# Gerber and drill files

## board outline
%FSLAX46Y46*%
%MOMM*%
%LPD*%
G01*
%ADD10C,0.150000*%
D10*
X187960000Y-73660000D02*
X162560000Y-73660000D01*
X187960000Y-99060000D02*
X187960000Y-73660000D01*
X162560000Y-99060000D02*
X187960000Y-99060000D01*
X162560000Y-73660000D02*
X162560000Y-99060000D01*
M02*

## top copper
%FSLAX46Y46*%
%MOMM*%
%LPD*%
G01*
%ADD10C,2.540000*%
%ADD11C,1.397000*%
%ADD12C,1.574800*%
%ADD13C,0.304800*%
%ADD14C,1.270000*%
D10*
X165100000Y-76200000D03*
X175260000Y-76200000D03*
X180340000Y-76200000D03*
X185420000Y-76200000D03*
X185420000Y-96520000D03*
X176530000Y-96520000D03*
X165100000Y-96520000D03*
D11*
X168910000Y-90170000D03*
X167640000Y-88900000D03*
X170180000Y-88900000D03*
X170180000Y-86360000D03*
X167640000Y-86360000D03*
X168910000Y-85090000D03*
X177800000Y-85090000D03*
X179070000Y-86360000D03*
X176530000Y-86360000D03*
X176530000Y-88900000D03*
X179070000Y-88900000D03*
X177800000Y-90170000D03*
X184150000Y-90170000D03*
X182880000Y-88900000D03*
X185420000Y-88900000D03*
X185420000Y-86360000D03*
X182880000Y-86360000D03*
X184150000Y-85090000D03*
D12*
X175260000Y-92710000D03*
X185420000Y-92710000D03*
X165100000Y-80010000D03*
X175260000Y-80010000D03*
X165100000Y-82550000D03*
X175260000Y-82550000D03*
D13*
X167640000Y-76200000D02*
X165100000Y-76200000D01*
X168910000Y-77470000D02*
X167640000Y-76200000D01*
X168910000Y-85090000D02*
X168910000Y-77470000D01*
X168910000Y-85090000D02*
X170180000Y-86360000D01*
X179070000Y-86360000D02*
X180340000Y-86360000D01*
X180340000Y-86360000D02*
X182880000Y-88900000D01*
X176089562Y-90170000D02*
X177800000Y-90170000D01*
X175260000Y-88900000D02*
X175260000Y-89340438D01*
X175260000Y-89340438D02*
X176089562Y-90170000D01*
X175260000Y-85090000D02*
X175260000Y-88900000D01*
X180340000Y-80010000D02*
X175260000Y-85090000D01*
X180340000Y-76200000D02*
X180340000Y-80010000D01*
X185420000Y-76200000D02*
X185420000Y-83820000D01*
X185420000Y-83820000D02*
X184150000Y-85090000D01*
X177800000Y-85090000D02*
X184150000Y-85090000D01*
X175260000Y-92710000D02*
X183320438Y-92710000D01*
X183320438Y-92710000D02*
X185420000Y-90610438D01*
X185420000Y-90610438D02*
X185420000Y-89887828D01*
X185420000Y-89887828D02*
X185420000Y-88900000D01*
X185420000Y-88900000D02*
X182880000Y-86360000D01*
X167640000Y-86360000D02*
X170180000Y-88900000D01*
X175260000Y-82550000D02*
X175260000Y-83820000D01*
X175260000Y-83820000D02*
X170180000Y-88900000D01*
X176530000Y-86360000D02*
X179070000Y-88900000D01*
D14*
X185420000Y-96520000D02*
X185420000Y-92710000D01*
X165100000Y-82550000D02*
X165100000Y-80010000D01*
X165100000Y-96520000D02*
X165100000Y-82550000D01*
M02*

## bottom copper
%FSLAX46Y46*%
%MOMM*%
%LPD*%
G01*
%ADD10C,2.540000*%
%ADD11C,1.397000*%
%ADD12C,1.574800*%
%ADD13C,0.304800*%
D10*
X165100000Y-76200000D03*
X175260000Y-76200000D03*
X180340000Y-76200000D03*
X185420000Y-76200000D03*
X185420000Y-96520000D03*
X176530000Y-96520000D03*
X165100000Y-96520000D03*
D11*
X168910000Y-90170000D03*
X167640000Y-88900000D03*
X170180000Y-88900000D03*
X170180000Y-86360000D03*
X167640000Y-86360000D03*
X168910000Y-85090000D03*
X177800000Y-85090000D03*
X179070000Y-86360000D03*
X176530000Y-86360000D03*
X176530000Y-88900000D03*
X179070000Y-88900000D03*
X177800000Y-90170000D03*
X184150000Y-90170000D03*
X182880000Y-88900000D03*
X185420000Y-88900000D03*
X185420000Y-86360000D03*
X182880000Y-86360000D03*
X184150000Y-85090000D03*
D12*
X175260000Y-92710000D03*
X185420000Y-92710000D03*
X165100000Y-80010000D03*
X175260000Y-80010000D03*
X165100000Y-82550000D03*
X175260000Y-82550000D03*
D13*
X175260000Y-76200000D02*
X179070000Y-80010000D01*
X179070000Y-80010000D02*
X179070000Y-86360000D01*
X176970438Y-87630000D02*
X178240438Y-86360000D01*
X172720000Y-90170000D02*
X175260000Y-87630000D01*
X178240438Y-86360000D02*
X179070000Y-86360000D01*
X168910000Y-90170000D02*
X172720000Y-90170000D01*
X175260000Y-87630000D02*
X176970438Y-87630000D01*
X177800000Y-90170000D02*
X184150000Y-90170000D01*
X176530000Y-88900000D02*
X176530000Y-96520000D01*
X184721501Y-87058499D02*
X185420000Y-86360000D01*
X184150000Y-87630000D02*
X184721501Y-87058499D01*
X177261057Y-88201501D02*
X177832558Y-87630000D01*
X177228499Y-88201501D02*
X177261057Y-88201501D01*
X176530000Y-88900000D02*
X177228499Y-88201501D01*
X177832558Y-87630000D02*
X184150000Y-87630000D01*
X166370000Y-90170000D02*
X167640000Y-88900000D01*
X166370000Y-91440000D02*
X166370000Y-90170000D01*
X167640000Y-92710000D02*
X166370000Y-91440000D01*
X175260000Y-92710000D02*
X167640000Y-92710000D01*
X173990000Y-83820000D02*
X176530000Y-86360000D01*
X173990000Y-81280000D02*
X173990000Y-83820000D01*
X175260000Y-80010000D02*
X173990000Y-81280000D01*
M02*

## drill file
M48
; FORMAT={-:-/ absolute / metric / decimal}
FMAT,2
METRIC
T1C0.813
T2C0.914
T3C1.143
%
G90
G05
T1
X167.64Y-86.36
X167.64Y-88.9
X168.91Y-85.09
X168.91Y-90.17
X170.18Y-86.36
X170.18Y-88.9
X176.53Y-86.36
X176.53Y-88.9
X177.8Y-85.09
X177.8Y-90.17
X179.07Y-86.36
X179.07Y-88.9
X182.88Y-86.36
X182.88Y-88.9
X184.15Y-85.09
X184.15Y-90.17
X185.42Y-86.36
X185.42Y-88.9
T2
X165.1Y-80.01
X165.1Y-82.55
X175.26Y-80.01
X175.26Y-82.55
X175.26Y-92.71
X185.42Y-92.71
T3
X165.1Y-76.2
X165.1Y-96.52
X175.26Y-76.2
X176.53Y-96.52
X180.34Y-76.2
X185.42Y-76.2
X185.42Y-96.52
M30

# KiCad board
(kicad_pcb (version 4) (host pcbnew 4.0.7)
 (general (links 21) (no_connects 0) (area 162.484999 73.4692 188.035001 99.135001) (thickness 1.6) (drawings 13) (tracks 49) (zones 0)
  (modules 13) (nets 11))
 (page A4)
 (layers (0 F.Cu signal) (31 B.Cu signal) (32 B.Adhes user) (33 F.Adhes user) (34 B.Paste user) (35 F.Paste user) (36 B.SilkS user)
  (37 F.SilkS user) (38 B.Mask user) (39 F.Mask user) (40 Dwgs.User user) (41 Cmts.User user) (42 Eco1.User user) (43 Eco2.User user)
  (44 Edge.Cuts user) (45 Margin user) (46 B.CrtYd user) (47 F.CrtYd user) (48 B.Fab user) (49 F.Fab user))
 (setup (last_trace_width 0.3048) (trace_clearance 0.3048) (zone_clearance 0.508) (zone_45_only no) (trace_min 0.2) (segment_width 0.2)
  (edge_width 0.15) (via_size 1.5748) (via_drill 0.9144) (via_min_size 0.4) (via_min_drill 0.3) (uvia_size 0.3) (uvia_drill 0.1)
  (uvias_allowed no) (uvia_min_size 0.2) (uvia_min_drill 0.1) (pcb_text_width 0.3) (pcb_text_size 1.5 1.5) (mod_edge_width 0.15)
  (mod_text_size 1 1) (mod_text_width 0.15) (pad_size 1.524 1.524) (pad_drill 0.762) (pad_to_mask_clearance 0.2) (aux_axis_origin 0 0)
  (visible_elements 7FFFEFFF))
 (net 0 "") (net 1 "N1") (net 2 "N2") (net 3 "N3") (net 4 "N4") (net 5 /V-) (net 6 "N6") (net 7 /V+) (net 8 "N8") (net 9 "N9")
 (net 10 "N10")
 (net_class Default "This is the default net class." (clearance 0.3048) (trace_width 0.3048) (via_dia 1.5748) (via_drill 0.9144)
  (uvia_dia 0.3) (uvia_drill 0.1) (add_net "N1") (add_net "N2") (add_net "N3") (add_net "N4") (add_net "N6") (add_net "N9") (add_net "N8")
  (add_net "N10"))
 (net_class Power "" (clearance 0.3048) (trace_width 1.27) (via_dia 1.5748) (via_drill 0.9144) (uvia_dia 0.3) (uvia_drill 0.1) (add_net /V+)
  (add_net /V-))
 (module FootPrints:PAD (layer F.Cu) (at 165.1 76.2)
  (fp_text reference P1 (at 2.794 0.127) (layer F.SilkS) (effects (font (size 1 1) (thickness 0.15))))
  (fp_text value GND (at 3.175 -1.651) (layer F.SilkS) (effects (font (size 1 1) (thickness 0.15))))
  (pad 1 thru_hole circle (at 0 0) (size 2.54 2.54) (drill 1.143) (layers *.Cu *.Mask F.SilkS) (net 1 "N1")))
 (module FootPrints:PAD (layer F.Cu) (at 175.26 76.2)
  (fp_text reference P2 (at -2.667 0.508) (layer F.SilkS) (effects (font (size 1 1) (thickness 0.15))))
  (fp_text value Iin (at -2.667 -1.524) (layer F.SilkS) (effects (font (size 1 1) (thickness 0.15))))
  (pad 1 thru_hole circle (at 0 0) (size 2.54 2.54) (drill 1.143) (layers *.Cu *.Mask F.SilkS) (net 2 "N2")))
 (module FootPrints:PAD (layer F.Cu) (at 180.34 76.2)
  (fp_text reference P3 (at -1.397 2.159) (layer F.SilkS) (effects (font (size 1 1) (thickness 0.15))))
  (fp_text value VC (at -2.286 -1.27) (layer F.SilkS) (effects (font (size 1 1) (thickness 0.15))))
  (pad 1 thru_hole circle (at 0 0) (size 2.54 2.54) (drill 1.143) (layers *.Cu *.Mask F.SilkS) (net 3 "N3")))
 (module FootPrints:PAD (layer F.Cu) (at 185.42 76.2)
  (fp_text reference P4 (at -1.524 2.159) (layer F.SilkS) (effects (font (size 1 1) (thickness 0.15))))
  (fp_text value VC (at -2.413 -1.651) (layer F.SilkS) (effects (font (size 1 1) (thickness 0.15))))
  (pad 1 thru_hole circle (at 0 0) (size 2.54 2.54) (drill 1.143) (layers *.Cu *.Mask F.SilkS) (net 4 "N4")))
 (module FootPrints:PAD (layer F.Cu) (at 185.42 96.52)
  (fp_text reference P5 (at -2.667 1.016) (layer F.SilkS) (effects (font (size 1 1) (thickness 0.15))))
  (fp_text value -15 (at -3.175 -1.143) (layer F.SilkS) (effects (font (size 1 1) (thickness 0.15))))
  (pad 1 thru_hole circle (at 0 0) (size 2.54 2.54) (drill 1.143) (layers *.Cu *.Mask F.SilkS) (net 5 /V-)))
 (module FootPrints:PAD (layer F.Cu) (at 176.53 96.52)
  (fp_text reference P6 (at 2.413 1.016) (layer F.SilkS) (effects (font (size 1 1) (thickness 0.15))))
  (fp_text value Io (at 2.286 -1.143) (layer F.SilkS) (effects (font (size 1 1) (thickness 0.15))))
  (pad 1 thru_hole circle (at 0 0) (size 2.54 2.54) (drill 1.143) (layers *.Cu *.Mask F.SilkS) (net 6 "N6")))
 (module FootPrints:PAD (layer F.Cu) (at 165.1 96.52)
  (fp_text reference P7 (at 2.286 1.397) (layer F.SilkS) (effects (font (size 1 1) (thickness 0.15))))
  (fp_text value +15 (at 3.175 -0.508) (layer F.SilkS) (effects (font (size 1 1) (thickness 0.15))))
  (pad 1 thru_hole circle (at 0 0) (size 2.54 2.54) (drill 1.143) (layers *.Cu *.Mask F.SilkS) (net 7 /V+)))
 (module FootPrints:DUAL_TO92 (layer F.Cu) (at 168.91 87.63)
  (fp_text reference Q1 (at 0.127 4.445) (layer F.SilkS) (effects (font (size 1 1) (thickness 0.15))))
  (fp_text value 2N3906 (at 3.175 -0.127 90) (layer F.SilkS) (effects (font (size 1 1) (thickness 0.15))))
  (pad 2 thru_hole circle (at 0 2.54) (size 1.397 1.397) (drill 0.8128) (layers *.Cu *.Mask F.SilkS) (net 2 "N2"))
  (pad 3 thru_hole circle (at -1.27 1.27) (size 1.397 1.397) (drill 0.8128) (layers *.Cu *.Mask F.SilkS) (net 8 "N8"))
  (pad 1 thru_hole circle (at 1.27 1.27) (size 1.397 1.397) (drill 0.8128) (layers *.Cu *.Mask F.SilkS) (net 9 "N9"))
  (pad 6 thru_hole circle (at 1.27 -1.27) (size 1.397 1.397) (drill 0.8128) (layers *.Cu *.Mask F.SilkS) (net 1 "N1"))
  (pad 4 thru_hole circle (at -1.27 -1.27) (size 1.397 1.397) (drill 0.8128) (layers *.Cu *.Mask F.SilkS) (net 9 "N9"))
  (pad 5 thru_hole circle (at 0 -2.54) (size 1.397 1.397) (drill 0.8128) (layers *.Cu *.Mask F.SilkS) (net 1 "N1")))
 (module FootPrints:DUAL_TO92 (layer F.Cu) (at 177.8 87.63 180)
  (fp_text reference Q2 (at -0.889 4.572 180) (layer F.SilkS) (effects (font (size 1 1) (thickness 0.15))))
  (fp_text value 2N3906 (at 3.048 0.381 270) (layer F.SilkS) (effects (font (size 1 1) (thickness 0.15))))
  (pad 2 thru_hole circle (at 0 2.54 180) (size 1.397 1.397) (drill 0.8128) (layers *.Cu *.Mask F.SilkS) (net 4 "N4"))
  (pad 3 thru_hole circle (at -1.27 1.27 180) (size 1.397 1.397) (drill 0.8128) (layers *.Cu *.Mask F.SilkS) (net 2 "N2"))
  (pad 1 thru_hole circle (at 1.27 1.27 180) (size 1.397 1.397) (drill 0.8128) (layers *.Cu *.Mask F.SilkS) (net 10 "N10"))
  (pad 6 thru_hole circle (at 1.27 -1.27 180) (size 1.397 1.397) (drill 0.8128) (layers *.Cu *.Mask F.SilkS) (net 6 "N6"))
  (pad 4 thru_hole circle (at -1.27 -1.27 180) (size 1.397 1.397) (drill 0.8128) (layers *.Cu *.Mask F.SilkS) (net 10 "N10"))
  (pad 5 thru_hole circle (at 0 -2.54 180) (size 1.397 1.397) (drill 0.8128) (layers *.Cu *.Mask F.SilkS) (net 3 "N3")))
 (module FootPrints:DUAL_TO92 (layer F.Cu) (at 184.15 87.63)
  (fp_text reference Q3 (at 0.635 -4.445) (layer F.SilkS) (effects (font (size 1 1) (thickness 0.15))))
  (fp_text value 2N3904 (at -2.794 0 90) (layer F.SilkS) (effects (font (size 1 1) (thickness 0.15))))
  (pad 2 thru_hole circle (at 0 2.54) (size 1.397 1.397) (drill 0.8128) (layers *.Cu *.Mask F.SilkS) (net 3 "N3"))
  (pad 3 thru_hole circle (at -1.27 1.27) (size 1.397 1.397) (drill 0.8128) (layers *.Cu *.Mask F.SilkS) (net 2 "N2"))
  (pad 1 thru_hole circle (at 1.27 1.27) (size 1.397 1.397) (drill 0.8128) (layers *.Cu *.Mask F.SilkS) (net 8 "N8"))
  (pad 6 thru_hole circle (at 1.27 -1.27) (size 1.397 1.397) (drill 0.8128) (layers *.Cu *.Mask F.SilkS) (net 6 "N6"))
  (pad 4 thru_hole circle (at -1.27 -1.27) (size 1.397 1.397) (drill 0.8128) (layers *.Cu *.Mask F.SilkS) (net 8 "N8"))
  (pad 5 thru_hole circle (at 0 -2.54) (size 1.397 1.397) (drill 0.8128) (layers *.Cu *.Mask F.SilkS) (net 4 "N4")))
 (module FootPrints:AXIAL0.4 (layer F.Cu) (at 180.34 92.71)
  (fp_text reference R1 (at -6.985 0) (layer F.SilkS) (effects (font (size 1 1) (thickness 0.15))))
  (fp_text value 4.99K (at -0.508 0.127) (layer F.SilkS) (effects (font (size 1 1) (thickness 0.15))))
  (pad 1 thru_hole circle (at -5.08 0) (size 1.5748 1.5748) (drill 0.9144) (layers *.Cu *.Mask F.SilkS) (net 8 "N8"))
  (pad 2 thru_hole circle (at 5.08 0) (size 1.5748 1.5748) (drill 0.9144) (layers *.Cu *.Mask F.SilkS) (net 5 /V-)))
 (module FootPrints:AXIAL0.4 (layer F.Cu) (at 170.18 80.01)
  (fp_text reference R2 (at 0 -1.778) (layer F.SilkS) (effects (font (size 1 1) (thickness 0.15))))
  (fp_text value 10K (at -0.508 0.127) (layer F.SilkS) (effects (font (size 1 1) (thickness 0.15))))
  (pad 1 thru_hole circle (at -5.08 0) (size 1.5748 1.5748) (drill 0.9144) (layers *.Cu *.Mask F.SilkS) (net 7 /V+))
  (pad 2 thru_hole circle (at 5.08 0) (size 1.5748 1.5748) (drill 0.9144) (layers *.Cu *.Mask F.SilkS) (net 10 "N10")))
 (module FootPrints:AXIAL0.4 (layer F.Cu) (at 170.18 82.55)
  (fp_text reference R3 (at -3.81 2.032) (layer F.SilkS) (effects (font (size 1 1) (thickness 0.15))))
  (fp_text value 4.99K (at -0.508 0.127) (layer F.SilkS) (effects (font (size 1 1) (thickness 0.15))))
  (pad 1 thru_hole circle (at -5.08 0) (size 1.5748 1.5748) (drill 0.9144) (layers *.Cu *.Mask F.SilkS) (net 7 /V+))
  (pad 2 thru_hole circle (at 5.08 0) (size 1.5748 1.5748) (drill 0.9144) (layers *.Cu *.Mask F.SilkS) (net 9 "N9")))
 (gr_line (start 187.96 73.66) (end 162.56 73.66) (layer Edge.Cuts) (width 0.15))
 (gr_line (start 187.96 99.06) (end 187.96 73.66) (layer Edge.Cuts) (width 0.15))
 (gr_line (start 162.56 99.06) (end 187.96 99.06) (layer Edge.Cuts) (width 0.15))
 (gr_line (start 162.56 73.66) (end 162.56 99.06) (layer Edge.Cuts) (width 0.15))
 (segment (start 167.64 76.2) (end 165.1 76.2) (width 0.3048) (layer F.Cu) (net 1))
 (segment (start 168.91 77.47) (end 167.64 76.2) (width 0.3048) (layer F.Cu) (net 1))
 (segment (start 168.91 85.09) (end 168.91 77.47) (width 0.3048) (layer F.Cu) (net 1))
 (segment (start 168.91 85.09) (end 170.18 86.36) (width 0.3048) (layer F.Cu) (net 1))
 (segment (start 175.26 76.2) (end 179.07 80.01) (width 0.3048) (layer B.Cu) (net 2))
 (segment (start 179.07 80.01) (end 179.07 86.36) (width 0.3048) (layer B.Cu) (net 2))
 (segment (start 179.07 86.36) (end 180.34 86.36) (width 0.3048) (layer F.Cu) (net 2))
 (segment (start 180.34 86.36) (end 182.88 88.9) (width 0.3048) (layer F.Cu) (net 2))
 (segment (start 176.970438 87.63) (end 178.240438 86.36) (width 0.3048) (layer B.Cu) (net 2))
 (segment (start 172.72 90.17) (end 175.26 87.63) (width 0.3048) (layer B.Cu) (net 2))
 (segment (start 178.240438 86.36) (end 179.07 86.36) (width 0.3048) (layer B.Cu) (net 2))
 (segment (start 168.91 90.17) (end 172.72 90.17) (width 0.3048) (layer B.Cu) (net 2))
 (segment (start 175.26 87.63) (end 176.970438 87.63) (width 0.3048) (layer B.Cu) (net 2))
 (segment (start 176.089562 90.17) (end 177.8 90.17) (width 0.3048) (layer F.Cu) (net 3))
 (segment (start 175.26 88.9) (end 175.26 89.340438) (width 0.3048) (layer F.Cu) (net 3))
 (segment (start 175.26 89.340438) (end 176.089562 90.17) (width 0.3048) (layer F.Cu) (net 3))
 (segment (start 175.26 85.09) (end 175.26 88.9) (width 0.3048) (layer F.Cu) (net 3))
 (segment (start 180.34 80.01) (end 175.26 85.09) (width 0.3048) (layer F.Cu) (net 3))
 (segment (start 180.34 76.2) (end 180.34 80.01) (width 0.3048) (layer F.Cu) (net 3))
 (segment (start 177.8 90.17) (end 184.15 90.17) (width 0.3048) (layer B.Cu) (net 3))
 (segment (start 185.42 76.2) (end 185.42 83.82) (width 0.3048) (layer F.Cu) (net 4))
 (segment (start 185.42 83.82) (end 184.15 85.09) (width 0.3048) (layer F.Cu) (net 4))
 (segment (start 177.8 85.09) (end 184.15 85.09) (width 0.3048) (layer F.Cu) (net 4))
 (segment (start 176.53 88.9) (end 176.53 96.52) (width 0.3048) (layer B.Cu) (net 6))
 (segment (start 184.721501 87.058499) (end 185.42 86.36) (width 0.3048) (layer B.Cu) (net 6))
 (segment (start 184.15 87.63) (end 184.721501 87.058499) (width 0.3048) (layer B.Cu) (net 6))
 (segment (start 177.261057 88.201501) (end 177.832558 87.63) (width 0.3048) (layer B.Cu) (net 6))
 (segment (start 177.228499 88.201501) (end 177.261057 88.201501) (width 0.3048) (layer B.Cu) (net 6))
 (segment (start 176.53 88.9) (end 177.228499 88.201501) (width 0.3048) (layer B.Cu) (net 6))
 (segment (start 177.832558 87.63) (end 184.15 87.63) (width 0.3048) (layer B.Cu) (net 6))
 (segment (start 175.26 92.71) (end 183.320438 92.71) (width 0.3048) (layer F.Cu) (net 8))
 (segment (start 183.320438 92.71) (end 185.42 90.610438) (width 0.3048) (layer F.Cu) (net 8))
 (segment (start 185.42 90.610438) (end 185.42 89.887828) (width 0.3048) (layer F.Cu) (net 8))
 (segment (start 185.42 89.887828) (end 185.42 88.9) (width 0.3048) (layer F.Cu) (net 8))
 (segment (start 166.37 90.17) (end 167.64 88.9) (width 0.3048) (layer B.Cu) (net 8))
 (segment (start 166.37 91.44) (end 166.37 90.17) (width 0.3048) (layer B.Cu) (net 8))
 (segment (start 167.64 92.71) (end 166.37 91.44) (width 0.3048) (layer B.Cu) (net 8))
 (segment (start 175.26 92.71) (end 167.64 92.71) (width 0.3048) (layer B.Cu) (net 8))
 (segment (start 185.42 88.9) (end 182.88 86.36) (width 0.3048) (layer F.Cu) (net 8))
 (segment (start 167.64 86.36) (end 170.18 88.9) (width 0.3048) (layer F.Cu) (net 9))
 (segment (start 175.26 82.55) (end 175.26 83.82) (width 0.3048) (layer F.Cu) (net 9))
 (segment (start 175.26 83.82) (end 170.18 88.9) (width 0.3048) (layer F.Cu) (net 9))
 (segment (start 173.99 83.82) (end 176.53 86.36) (width 0.3048) (layer B.Cu) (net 10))
 (segment (start 173.99 81.28) (end 173.99 83.82) (width 0.3048) (layer B.Cu) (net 10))
 (segment (start 175.26 80.01) (end 173.99 81.28) (width 0.3048) (layer B.Cu) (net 10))
 (segment (start 176.53 86.36) (end 179.07 88.9) (width 0.3048) (layer F.Cu) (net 10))
 (segment (start 185.42 96.52) (end 185.42 92.71) (width 1.27) (layer F.Cu) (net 5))
 (segment (start 165.1 82.55) (end 165.1 80.01) (width 1.27) (layer F.Cu) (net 7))
 (segment (start 165.1 96.52) (end 165.1 82.55) (width 1.27) (layer F.Cu) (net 7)))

